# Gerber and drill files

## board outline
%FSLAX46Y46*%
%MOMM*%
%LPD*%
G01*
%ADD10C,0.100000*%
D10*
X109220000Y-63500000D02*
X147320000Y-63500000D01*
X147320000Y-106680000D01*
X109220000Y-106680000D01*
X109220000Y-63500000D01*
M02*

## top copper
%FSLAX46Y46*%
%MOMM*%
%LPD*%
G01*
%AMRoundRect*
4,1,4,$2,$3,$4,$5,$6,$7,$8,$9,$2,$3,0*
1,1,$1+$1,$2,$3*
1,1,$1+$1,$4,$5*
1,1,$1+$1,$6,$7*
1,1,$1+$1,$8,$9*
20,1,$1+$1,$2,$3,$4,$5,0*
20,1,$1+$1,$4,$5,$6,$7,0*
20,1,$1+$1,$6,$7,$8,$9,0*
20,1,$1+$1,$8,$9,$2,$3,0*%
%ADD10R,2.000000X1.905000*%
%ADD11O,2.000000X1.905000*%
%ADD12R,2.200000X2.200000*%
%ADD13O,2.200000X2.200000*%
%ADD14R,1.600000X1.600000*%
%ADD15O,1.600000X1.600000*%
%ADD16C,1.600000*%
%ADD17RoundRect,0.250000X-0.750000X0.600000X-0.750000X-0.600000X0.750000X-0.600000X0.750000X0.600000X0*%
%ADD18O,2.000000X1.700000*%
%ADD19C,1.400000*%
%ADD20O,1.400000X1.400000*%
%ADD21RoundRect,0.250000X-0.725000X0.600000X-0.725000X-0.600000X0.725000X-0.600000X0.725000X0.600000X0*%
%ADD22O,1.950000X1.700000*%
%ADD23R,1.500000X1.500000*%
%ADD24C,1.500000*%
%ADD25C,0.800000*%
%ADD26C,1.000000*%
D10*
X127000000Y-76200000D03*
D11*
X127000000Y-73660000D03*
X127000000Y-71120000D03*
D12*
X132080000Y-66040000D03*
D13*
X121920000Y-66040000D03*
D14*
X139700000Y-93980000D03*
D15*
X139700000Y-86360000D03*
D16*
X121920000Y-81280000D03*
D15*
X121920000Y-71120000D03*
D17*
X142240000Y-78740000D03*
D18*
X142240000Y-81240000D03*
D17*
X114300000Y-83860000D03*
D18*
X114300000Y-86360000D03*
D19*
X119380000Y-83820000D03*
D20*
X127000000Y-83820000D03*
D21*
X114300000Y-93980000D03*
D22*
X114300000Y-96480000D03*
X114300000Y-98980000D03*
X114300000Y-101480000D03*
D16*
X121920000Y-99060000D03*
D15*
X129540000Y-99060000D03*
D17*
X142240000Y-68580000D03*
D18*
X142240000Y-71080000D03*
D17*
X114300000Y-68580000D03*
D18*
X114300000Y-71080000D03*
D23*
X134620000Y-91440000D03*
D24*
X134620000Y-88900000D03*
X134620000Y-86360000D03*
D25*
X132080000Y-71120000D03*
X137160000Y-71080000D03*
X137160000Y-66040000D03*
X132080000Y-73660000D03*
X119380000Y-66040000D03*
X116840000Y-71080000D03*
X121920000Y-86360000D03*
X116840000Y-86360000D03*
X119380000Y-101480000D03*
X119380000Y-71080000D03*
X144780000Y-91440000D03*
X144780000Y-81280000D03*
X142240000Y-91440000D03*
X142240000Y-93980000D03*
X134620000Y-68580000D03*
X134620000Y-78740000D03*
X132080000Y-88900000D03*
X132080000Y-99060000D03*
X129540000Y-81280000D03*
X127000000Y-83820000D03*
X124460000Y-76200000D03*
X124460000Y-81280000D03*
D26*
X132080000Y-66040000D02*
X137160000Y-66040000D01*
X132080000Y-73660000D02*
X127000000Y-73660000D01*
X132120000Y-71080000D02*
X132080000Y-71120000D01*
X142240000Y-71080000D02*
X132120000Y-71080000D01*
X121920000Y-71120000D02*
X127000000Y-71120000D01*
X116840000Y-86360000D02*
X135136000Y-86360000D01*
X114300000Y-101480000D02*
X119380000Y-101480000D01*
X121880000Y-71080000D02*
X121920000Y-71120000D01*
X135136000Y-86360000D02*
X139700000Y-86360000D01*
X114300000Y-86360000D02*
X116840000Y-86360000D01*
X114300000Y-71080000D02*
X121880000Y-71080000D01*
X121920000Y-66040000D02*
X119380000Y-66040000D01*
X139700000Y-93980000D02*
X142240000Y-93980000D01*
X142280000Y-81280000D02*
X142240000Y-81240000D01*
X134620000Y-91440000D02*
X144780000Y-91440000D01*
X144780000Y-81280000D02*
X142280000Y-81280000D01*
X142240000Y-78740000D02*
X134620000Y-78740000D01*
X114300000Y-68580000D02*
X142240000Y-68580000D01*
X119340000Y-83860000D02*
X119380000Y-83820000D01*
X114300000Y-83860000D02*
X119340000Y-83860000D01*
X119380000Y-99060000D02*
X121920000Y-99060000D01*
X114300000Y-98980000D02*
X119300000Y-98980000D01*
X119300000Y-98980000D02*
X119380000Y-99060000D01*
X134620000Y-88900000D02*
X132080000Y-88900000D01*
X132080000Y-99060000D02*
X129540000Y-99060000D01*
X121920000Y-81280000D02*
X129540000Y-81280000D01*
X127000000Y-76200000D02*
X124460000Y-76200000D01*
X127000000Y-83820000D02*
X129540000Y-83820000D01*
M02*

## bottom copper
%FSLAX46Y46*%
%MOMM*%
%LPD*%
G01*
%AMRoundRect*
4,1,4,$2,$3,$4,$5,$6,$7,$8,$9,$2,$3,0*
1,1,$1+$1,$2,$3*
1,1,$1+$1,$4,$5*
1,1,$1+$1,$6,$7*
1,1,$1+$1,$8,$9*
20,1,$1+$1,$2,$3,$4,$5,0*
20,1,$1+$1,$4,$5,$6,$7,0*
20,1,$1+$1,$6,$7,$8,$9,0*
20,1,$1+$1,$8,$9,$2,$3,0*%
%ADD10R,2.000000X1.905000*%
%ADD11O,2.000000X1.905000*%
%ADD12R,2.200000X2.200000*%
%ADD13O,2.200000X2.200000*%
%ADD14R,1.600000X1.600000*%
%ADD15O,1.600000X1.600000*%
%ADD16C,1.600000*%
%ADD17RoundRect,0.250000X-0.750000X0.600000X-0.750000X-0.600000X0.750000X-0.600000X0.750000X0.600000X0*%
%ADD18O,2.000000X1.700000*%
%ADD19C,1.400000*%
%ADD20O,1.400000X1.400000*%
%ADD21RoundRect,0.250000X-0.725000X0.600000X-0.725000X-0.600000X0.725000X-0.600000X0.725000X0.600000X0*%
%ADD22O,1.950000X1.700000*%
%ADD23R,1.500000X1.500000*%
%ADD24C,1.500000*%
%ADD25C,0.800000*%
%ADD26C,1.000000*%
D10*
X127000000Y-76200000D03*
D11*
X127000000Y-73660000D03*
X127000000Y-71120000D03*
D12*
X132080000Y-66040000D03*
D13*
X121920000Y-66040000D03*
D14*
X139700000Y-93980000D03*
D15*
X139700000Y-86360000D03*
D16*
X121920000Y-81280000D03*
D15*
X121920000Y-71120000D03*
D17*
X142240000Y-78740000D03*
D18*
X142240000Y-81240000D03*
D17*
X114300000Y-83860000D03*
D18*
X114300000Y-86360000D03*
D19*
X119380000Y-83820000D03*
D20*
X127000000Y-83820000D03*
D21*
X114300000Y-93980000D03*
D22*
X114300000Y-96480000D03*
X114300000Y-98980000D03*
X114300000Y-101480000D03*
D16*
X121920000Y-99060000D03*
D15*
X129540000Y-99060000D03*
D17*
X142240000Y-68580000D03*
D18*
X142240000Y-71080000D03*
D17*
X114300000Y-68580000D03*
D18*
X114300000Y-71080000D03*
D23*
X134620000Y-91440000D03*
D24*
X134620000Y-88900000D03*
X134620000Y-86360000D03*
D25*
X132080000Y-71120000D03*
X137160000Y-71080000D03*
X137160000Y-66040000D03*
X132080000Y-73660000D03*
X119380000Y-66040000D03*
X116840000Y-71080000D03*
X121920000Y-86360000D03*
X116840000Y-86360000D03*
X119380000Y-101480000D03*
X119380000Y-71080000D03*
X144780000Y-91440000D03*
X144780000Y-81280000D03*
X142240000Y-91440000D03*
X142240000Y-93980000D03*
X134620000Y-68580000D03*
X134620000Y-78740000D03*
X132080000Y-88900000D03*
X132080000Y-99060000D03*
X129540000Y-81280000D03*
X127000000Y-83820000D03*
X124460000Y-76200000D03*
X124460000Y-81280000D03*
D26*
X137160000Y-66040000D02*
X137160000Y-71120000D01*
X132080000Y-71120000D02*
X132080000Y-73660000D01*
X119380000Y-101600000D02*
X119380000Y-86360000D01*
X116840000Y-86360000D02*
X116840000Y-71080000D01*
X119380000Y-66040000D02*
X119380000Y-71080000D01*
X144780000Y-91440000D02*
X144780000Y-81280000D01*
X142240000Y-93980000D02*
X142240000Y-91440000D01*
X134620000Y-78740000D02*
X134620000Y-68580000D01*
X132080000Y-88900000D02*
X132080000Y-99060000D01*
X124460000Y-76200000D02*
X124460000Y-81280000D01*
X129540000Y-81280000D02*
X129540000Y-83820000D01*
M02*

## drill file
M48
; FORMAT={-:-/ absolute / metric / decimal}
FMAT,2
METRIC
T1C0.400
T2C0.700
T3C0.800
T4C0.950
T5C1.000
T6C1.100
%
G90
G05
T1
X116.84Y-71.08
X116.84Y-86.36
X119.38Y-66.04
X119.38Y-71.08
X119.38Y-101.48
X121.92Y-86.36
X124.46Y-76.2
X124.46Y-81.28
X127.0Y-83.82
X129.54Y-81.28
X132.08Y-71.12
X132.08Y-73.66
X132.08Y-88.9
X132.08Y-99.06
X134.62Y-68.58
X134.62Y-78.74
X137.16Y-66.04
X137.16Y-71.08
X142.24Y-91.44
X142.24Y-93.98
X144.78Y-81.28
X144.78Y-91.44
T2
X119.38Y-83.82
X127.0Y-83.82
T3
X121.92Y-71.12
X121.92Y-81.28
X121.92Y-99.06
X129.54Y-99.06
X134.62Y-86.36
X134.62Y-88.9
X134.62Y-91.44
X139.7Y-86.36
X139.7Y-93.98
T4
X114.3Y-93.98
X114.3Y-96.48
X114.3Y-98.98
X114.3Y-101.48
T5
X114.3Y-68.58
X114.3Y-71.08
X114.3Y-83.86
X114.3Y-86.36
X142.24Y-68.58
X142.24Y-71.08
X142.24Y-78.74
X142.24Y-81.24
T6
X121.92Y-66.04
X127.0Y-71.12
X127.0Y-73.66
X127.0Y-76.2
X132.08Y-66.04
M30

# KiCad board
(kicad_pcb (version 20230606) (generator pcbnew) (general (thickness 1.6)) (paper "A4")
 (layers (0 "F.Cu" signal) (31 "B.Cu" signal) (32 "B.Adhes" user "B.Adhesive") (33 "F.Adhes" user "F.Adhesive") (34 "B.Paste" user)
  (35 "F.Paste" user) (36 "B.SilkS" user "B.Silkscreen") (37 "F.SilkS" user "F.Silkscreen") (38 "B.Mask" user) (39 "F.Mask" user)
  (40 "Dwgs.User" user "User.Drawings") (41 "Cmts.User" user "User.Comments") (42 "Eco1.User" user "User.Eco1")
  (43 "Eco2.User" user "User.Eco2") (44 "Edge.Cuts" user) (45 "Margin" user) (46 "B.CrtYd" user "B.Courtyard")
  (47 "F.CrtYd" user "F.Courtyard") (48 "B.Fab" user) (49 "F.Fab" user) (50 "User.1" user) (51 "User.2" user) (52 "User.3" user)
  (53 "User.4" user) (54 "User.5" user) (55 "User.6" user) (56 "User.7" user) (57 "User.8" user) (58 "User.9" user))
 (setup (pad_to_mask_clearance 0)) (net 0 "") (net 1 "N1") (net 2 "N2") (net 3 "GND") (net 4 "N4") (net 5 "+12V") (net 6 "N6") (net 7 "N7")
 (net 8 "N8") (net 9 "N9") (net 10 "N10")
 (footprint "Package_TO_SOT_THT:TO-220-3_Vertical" (layer "F.Cu") (at 127 76.2 90)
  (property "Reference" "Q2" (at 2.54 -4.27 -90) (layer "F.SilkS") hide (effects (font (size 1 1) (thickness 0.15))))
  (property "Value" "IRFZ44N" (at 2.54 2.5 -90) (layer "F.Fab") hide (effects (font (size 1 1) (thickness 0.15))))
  (pad "1" thru_hole rect (at 0 0 90) (size 1.905 2) (drill 1.1) (layers "*.Cu" "*.Mask") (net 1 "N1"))
  (pad "2" thru_hole oval (at 2.54 0 90) (size 1.905 2) (drill 1.1) (layers "*.Cu" "*.Mask") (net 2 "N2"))
  (pad "3" thru_hole oval (at 5.08 0 90) (size 1.905 2) (drill 1.1) (layers "*.Cu" "*.Mask") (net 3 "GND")))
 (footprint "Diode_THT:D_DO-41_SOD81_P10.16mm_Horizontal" (layer "F.Cu") (at 132.08 66.04 180)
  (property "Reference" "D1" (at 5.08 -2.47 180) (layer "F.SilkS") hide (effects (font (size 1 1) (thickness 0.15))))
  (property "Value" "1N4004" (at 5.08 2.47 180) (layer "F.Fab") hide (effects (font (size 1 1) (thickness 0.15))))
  (pad "1" thru_hole rect (at 0 0 180) (size 2.2 2.2) (drill 1.1) (layers "*.Cu" "*.Mask") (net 2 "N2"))
  (pad "2" thru_hole oval (at 10.16 0 180) (size 2.2 2.2) (drill 1.1) (layers "*.Cu" "*.Mask") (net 3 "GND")))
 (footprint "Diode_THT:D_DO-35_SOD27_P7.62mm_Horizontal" (layer "F.Cu") (at 139.7 93.98 90)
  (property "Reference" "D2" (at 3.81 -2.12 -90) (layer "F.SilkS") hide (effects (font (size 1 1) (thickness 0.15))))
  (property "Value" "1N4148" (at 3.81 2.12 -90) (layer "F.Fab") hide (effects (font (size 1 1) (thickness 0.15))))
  (pad "1" thru_hole rect (at 0 0 90) (size 1.6 1.6) (drill 0.8) (layers "*.Cu" "*.Mask") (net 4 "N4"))
  (pad "2" thru_hole oval (at 7.62 0 90) (size 1.6 1.6) (drill 0.8) (layers "*.Cu" "*.Mask") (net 3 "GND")))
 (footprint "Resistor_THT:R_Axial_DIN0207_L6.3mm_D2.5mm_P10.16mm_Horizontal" (layer "F.Cu") (at 121.92 81.28 90)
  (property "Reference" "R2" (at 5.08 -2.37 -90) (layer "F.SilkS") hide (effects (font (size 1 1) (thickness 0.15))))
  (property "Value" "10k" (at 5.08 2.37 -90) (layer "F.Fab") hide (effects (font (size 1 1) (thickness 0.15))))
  (pad "1" thru_hole circle (at 0 0 90) (size 1.6 1.6) (drill 0.8) (layers "*.Cu" "*.Mask") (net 1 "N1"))
  (pad "2" thru_hole oval (at 10.16 0 90) (size 1.6 1.6) (drill 0.8) (layers "*.Cu" "*.Mask") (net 3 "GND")))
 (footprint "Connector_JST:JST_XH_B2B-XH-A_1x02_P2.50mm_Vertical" (layer "F.Cu") (at 142.24 78.74 -90)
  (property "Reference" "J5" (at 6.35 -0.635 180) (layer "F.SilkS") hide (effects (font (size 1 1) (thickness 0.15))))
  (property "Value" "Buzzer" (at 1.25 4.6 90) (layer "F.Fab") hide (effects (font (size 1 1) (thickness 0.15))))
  (pad "1" thru_hole roundrect (at 0 0 270) (size 1.7 2) (drill 1) (layers "*.Cu" "*.Mask") (roundrect_rratio 0.147059) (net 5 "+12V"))
  (pad "2" thru_hole oval (at 2.5 0 270) (size 1.7 2) (drill 1) (layers "*.Cu" "*.Mask") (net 4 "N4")))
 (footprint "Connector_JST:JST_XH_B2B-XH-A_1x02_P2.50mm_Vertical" (layer "F.Cu") (at 114.3 83.86 -90)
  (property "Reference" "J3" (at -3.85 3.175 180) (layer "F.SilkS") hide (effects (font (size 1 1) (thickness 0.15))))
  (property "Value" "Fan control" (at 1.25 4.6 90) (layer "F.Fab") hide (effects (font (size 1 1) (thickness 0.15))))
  (pad "1" thru_hole roundrect (at 0 0 270) (size 1.7 2) (drill 1) (layers "*.Cu" "*.Mask") (roundrect_rratio 0.147059) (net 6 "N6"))
  (pad "2" thru_hole oval (at 2.5 0 270) (size 1.7 2) (drill 1) (layers "*.Cu" "*.Mask") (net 3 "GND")))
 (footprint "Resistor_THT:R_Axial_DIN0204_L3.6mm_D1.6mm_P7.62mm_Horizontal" (layer "F.Cu") (at 119.38 83.82)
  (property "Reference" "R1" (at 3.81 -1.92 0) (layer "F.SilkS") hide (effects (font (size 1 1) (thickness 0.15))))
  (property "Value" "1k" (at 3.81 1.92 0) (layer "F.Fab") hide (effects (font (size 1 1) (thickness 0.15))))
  (pad "1" thru_hole circle (at 0 0) (size 1.4 1.4) (drill 0.7) (layers "*.Cu" "*.Mask") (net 6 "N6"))
  (pad "2" thru_hole oval (at 7.62 0) (size 1.4 1.4) (drill 0.7) (layers "*.Cu" "*.Mask") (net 1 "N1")))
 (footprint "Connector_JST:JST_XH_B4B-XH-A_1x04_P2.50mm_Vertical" (layer "F.Cu") (at 114.3 93.98 -90)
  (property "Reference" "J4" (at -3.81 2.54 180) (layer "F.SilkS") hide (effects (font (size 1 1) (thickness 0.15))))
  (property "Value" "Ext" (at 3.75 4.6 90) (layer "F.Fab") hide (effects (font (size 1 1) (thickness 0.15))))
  (pad "1" thru_hole roundrect (at 0 0 270) (size 1.7 1.95) (drill 0.95) (layers "*.Cu" "*.Mask") (roundrect_rratio 0.147059) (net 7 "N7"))
  (pad "2" thru_hole oval (at 2.5 0 270) (size 1.7 1.95) (drill 0.95) (layers "*.Cu" "*.Mask") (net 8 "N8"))
  (pad "3" thru_hole oval (at 5 0 270) (size 1.7 1.95) (drill 0.95) (layers "*.Cu" "*.Mask") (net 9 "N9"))
  (pad "4" thru_hole oval (at 7.5 0 270) (size 1.7 1.95) (drill 0.95) (layers "*.Cu" "*.Mask") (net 3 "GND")))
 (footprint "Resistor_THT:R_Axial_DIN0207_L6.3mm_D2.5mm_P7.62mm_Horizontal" (layer "F.Cu") (at 121.92 99.06)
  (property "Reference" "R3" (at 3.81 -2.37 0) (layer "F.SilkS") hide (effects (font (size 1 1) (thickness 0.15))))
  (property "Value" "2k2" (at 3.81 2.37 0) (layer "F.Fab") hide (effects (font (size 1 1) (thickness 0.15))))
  (pad "1" thru_hole circle (at 0 0) (size 1.6 1.6) (drill 0.8) (layers "*.Cu" "*.Mask") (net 9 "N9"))
  (pad "2" thru_hole oval (at 7.62 0) (size 1.6 1.6) (drill 0.8) (layers "*.Cu" "*.Mask") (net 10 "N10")))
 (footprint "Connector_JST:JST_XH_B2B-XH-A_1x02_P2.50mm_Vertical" (layer "F.Cu") (at 142.24 68.58 -90)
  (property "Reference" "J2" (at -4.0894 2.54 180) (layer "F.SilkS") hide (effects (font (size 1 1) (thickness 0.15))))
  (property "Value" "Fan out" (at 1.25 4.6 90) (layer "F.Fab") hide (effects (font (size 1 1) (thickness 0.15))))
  (pad "1" thru_hole roundrect (at 0 0 270) (size 1.7 2) (drill 1) (layers "*.Cu" "*.Mask") (roundrect_rratio 0.147059) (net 5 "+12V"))
  (pad "2" thru_hole oval (at 2.5 0 270) (size 1.7 2) (drill 1) (layers "*.Cu" "*.Mask") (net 2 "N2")))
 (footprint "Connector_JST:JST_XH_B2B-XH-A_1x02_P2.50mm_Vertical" (layer "F.Cu") (at 114.3 68.58 -90)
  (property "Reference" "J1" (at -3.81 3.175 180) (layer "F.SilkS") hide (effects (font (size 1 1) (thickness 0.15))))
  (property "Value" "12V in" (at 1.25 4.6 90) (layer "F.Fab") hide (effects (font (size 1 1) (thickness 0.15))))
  (pad "1" thru_hole roundrect (at 0 0 270) (size 1.7 2) (drill 1) (layers "*.Cu" "*.Mask") (roundrect_rratio 0.147059) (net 5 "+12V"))
  (pad "2" thru_hole oval (at 2.5 0 270) (size 1.7 2) (drill 1) (layers "*.Cu" "*.Mask") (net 3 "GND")))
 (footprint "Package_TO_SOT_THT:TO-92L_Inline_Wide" (layer "F.Cu") (at 134.62 91.44 90)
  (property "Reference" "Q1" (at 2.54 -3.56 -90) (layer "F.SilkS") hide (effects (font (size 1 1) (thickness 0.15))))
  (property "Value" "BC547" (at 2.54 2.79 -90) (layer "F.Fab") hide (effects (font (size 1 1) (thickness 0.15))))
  (pad "1" thru_hole rect (at 0 0 90) (size 1.5 1.5) (drill 0.8) (layers "*.Cu" "*.Mask") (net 4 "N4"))
  (pad "2" thru_hole circle (at 2.54 0 90) (size 1.5 1.5) (drill 0.8) (layers "*.Cu" "*.Mask") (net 10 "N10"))
  (pad "3" thru_hole circle (at 5.08 0 90) (size 1.5 1.5) (drill 0.8) (layers "*.Cu" "*.Mask") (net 3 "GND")))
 (gr_rect (start 109.22 63.5) (end 147.32 106.68) (stroke (width 0.1) (type default)) (fill none) (layer "Edge.Cuts"))
 (segment (start 132.08 66.04) (end 137.16 66.04) (width 1) (layer "F.Cu") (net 2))
 (segment (start 132.08 73.66) (end 127 73.66) (width 1) (layer "F.Cu") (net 2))
 (segment (start 132.12 71.08) (end 132.08 71.12) (width 1) (layer "F.Cu") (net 2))
 (segment (start 142.24 71.08) (end 132.12 71.08) (width 1) (layer "F.Cu") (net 2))
 (via (at 132.08 71.12) (size 0.8) (drill 0.4) (layers "F.Cu" "B.Cu") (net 2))
 (via (at 137.16 71.08) (size 0.8) (drill 0.4) (layers "F.Cu" "B.Cu") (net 2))
 (via (at 137.16 66.04) (size 0.8) (drill 0.4) (layers "F.Cu" "B.Cu") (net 2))
 (via (at 132.08 73.66) (size 0.8) (drill 0.4) (layers "F.Cu" "B.Cu") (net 2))
 (segment (start 137.16 66.04) (end 137.16 71.12) (width 1) (layer "B.Cu") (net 2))
 (segment (start 132.08 71.12) (end 132.08 73.66) (width 1) (layer "B.Cu") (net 2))
 (segment (start 121.92 71.12) (end 127 71.12) (width 1) (layer "F.Cu") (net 3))
 (segment (start 116.84 86.36) (end 135.136 86.36) (width 1) (layer "F.Cu") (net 3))
 (segment (start 114.3 101.48) (end 119.38 101.48) (width 1) (layer "F.Cu") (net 3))
 (segment (start 121.88 71.08) (end 121.92 71.12) (width 1) (layer "F.Cu") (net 3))
 (segment (start 135.136 86.36) (end 139.7 86.36) (width 1) (layer "F.Cu") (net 3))
 (segment (start 114.3 86.36) (end 116.84 86.36) (width 1) (layer "F.Cu") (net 3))
 (segment (start 114.3 71.08) (end 121.88 71.08) (width 1) (layer "F.Cu") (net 3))
 (segment (start 121.92 66.04) (end 119.38 66.04) (width 1) (layer "F.Cu") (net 3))
 (via (at 119.38 66.04) (size 0.8) (drill 0.4) (layers "F.Cu" "B.Cu") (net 3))
 (via (at 116.84 71.08) (size 0.8) (drill 0.4) (layers "F.Cu" "B.Cu") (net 3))
 (via (at 121.92 86.36) (size 0.8) (drill 0.4) (layers "F.Cu" "B.Cu") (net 3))
 (via (at 116.84 86.36) (size 0.8) (drill 0.4) (layers "F.Cu" "B.Cu") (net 3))
 (via (at 119.38 101.48) (size 0.8) (drill 0.4) (layers "F.Cu" "B.Cu") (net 3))
 (via (at 119.38 71.08) (size 0.8) (drill 0.4) (layers "F.Cu" "B.Cu") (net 3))
 (segment (start 119.38 101.6) (end 119.38 86.36) (width 1) (layer "B.Cu") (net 3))
 (segment (start 116.84 86.36) (end 116.84 71.08) (width 1) (layer "B.Cu") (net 3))
 (segment (start 119.38 66.04) (end 119.38 71.08) (width 1) (layer "B.Cu") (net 3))
 (segment (start 139.7 93.98) (end 142.24 93.98) (width 1) (layer "F.Cu") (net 4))
 (segment (start 142.28 81.28) (end 142.24 81.24) (width 1) (layer "F.Cu") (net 4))
 (segment (start 134.62 91.44) (end 144.78 91.44) (width 1) (layer "F.Cu") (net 4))
 (segment (start 144.78 81.28) (end 142.28 81.28) (width 1) (layer "F.Cu") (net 4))
 (via (at 144.78 91.44) (size 0.8) (drill 0.4) (layers "F.Cu" "B.Cu") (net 4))
 (via (at 144.78 81.28) (size 0.8) (drill 0.4) (layers "F.Cu" "B.Cu") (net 4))
 (via (at 142.24 91.44) (size 0.8) (drill 0.4) (layers "F.Cu" "B.Cu") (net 4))
 (via (at 142.24 93.98) (size 0.8) (drill 0.4) (layers "F.Cu" "B.Cu") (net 4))
 (segment (start 144.78 91.44) (end 144.78 81.28) (width 1) (layer "B.Cu") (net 4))
 (segment (start 142.24 93.98) (end 142.24 91.44) (width 1) (layer "B.Cu") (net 4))
 (segment (start 142.24 78.74) (end 134.62 78.74) (width 1) (layer "F.Cu") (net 5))
 (segment (start 114.3 68.58) (end 142.24 68.58) (width 1) (layer "F.Cu") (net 5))
 (via (at 134.62 68.58) (size 0.8) (drill 0.4) (layers "F.Cu" "B.Cu") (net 5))
 (via (at 134.62 78.74) (size 0.8) (drill 0.4) (layers "F.Cu" "B.Cu") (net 5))
 (segment (start 134.62 78.74) (end 134.62 68.58) (width 1) (layer "B.Cu") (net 5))
 (segment (start 119.34 83.86) (end 119.38 83.82) (width 1) (layer "F.Cu") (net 6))
 (segment (start 114.3 83.86) (end 119.34 83.86) (width 1) (layer "F.Cu") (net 6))
 (segment (start 119.38 99.06) (end 121.92 99.06) (width 1) (layer "F.Cu") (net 9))
 (segment (start 114.3 98.98) (end 119.3 98.98) (width 1) (layer "F.Cu") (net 9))
 (segment (start 119.3 98.98) (end 119.38 99.06) (width 1) (layer "F.Cu") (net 9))
 (segment (start 134.62 88.9) (end 132.08 88.9) (width 1) (layer "F.Cu") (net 10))
 (segment (start 132.08 99.06) (end 129.54 99.06) (width 1) (layer "F.Cu") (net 10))
 (via (at 132.08 88.9) (size 0.8) (drill 0.4) (layers "F.Cu" "B.Cu") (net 10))
 (via (at 132.08 99.06) (size 0.8) (drill 0.4) (layers "F.Cu" "B.Cu") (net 10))
 (segment (start 132.08 88.9) (end 132.08 99.06) (width 1) (layer "B.Cu") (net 10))
 (segment (start 121.92 81.28) (end 129.54 81.28) (width 1) (layer "F.Cu") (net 1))
 (segment (start 127 76.2) (end 124.46 76.2) (width 1) (layer "F.Cu") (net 1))
 (segment (start 127 83.82) (end 129.54 83.82) (width 1) (layer "F.Cu") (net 1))
 (via (at 129.54 81.28) (size 0.8) (drill 0.4) (layers "F.Cu" "B.Cu") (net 1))
 (via (at 127 83.82) (size 0.8) (drill 0.4) (layers "F.Cu" "B.Cu") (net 1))
 (via (at 124.46 76.2) (size 0.8) (drill 0.4) (layers "F.Cu" "B.Cu") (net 1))
 (via (at 124.46 81.28) (size 0.8) (drill 0.4) (layers "F.Cu" "B.Cu") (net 1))
 (segment (start 124.46 76.2) (end 124.46 81.28) (width 1) (layer "B.Cu") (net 1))
 (segment (start 129.54 81.28) (end 129.54 83.82) (width 1) (layer "B.Cu") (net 1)))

